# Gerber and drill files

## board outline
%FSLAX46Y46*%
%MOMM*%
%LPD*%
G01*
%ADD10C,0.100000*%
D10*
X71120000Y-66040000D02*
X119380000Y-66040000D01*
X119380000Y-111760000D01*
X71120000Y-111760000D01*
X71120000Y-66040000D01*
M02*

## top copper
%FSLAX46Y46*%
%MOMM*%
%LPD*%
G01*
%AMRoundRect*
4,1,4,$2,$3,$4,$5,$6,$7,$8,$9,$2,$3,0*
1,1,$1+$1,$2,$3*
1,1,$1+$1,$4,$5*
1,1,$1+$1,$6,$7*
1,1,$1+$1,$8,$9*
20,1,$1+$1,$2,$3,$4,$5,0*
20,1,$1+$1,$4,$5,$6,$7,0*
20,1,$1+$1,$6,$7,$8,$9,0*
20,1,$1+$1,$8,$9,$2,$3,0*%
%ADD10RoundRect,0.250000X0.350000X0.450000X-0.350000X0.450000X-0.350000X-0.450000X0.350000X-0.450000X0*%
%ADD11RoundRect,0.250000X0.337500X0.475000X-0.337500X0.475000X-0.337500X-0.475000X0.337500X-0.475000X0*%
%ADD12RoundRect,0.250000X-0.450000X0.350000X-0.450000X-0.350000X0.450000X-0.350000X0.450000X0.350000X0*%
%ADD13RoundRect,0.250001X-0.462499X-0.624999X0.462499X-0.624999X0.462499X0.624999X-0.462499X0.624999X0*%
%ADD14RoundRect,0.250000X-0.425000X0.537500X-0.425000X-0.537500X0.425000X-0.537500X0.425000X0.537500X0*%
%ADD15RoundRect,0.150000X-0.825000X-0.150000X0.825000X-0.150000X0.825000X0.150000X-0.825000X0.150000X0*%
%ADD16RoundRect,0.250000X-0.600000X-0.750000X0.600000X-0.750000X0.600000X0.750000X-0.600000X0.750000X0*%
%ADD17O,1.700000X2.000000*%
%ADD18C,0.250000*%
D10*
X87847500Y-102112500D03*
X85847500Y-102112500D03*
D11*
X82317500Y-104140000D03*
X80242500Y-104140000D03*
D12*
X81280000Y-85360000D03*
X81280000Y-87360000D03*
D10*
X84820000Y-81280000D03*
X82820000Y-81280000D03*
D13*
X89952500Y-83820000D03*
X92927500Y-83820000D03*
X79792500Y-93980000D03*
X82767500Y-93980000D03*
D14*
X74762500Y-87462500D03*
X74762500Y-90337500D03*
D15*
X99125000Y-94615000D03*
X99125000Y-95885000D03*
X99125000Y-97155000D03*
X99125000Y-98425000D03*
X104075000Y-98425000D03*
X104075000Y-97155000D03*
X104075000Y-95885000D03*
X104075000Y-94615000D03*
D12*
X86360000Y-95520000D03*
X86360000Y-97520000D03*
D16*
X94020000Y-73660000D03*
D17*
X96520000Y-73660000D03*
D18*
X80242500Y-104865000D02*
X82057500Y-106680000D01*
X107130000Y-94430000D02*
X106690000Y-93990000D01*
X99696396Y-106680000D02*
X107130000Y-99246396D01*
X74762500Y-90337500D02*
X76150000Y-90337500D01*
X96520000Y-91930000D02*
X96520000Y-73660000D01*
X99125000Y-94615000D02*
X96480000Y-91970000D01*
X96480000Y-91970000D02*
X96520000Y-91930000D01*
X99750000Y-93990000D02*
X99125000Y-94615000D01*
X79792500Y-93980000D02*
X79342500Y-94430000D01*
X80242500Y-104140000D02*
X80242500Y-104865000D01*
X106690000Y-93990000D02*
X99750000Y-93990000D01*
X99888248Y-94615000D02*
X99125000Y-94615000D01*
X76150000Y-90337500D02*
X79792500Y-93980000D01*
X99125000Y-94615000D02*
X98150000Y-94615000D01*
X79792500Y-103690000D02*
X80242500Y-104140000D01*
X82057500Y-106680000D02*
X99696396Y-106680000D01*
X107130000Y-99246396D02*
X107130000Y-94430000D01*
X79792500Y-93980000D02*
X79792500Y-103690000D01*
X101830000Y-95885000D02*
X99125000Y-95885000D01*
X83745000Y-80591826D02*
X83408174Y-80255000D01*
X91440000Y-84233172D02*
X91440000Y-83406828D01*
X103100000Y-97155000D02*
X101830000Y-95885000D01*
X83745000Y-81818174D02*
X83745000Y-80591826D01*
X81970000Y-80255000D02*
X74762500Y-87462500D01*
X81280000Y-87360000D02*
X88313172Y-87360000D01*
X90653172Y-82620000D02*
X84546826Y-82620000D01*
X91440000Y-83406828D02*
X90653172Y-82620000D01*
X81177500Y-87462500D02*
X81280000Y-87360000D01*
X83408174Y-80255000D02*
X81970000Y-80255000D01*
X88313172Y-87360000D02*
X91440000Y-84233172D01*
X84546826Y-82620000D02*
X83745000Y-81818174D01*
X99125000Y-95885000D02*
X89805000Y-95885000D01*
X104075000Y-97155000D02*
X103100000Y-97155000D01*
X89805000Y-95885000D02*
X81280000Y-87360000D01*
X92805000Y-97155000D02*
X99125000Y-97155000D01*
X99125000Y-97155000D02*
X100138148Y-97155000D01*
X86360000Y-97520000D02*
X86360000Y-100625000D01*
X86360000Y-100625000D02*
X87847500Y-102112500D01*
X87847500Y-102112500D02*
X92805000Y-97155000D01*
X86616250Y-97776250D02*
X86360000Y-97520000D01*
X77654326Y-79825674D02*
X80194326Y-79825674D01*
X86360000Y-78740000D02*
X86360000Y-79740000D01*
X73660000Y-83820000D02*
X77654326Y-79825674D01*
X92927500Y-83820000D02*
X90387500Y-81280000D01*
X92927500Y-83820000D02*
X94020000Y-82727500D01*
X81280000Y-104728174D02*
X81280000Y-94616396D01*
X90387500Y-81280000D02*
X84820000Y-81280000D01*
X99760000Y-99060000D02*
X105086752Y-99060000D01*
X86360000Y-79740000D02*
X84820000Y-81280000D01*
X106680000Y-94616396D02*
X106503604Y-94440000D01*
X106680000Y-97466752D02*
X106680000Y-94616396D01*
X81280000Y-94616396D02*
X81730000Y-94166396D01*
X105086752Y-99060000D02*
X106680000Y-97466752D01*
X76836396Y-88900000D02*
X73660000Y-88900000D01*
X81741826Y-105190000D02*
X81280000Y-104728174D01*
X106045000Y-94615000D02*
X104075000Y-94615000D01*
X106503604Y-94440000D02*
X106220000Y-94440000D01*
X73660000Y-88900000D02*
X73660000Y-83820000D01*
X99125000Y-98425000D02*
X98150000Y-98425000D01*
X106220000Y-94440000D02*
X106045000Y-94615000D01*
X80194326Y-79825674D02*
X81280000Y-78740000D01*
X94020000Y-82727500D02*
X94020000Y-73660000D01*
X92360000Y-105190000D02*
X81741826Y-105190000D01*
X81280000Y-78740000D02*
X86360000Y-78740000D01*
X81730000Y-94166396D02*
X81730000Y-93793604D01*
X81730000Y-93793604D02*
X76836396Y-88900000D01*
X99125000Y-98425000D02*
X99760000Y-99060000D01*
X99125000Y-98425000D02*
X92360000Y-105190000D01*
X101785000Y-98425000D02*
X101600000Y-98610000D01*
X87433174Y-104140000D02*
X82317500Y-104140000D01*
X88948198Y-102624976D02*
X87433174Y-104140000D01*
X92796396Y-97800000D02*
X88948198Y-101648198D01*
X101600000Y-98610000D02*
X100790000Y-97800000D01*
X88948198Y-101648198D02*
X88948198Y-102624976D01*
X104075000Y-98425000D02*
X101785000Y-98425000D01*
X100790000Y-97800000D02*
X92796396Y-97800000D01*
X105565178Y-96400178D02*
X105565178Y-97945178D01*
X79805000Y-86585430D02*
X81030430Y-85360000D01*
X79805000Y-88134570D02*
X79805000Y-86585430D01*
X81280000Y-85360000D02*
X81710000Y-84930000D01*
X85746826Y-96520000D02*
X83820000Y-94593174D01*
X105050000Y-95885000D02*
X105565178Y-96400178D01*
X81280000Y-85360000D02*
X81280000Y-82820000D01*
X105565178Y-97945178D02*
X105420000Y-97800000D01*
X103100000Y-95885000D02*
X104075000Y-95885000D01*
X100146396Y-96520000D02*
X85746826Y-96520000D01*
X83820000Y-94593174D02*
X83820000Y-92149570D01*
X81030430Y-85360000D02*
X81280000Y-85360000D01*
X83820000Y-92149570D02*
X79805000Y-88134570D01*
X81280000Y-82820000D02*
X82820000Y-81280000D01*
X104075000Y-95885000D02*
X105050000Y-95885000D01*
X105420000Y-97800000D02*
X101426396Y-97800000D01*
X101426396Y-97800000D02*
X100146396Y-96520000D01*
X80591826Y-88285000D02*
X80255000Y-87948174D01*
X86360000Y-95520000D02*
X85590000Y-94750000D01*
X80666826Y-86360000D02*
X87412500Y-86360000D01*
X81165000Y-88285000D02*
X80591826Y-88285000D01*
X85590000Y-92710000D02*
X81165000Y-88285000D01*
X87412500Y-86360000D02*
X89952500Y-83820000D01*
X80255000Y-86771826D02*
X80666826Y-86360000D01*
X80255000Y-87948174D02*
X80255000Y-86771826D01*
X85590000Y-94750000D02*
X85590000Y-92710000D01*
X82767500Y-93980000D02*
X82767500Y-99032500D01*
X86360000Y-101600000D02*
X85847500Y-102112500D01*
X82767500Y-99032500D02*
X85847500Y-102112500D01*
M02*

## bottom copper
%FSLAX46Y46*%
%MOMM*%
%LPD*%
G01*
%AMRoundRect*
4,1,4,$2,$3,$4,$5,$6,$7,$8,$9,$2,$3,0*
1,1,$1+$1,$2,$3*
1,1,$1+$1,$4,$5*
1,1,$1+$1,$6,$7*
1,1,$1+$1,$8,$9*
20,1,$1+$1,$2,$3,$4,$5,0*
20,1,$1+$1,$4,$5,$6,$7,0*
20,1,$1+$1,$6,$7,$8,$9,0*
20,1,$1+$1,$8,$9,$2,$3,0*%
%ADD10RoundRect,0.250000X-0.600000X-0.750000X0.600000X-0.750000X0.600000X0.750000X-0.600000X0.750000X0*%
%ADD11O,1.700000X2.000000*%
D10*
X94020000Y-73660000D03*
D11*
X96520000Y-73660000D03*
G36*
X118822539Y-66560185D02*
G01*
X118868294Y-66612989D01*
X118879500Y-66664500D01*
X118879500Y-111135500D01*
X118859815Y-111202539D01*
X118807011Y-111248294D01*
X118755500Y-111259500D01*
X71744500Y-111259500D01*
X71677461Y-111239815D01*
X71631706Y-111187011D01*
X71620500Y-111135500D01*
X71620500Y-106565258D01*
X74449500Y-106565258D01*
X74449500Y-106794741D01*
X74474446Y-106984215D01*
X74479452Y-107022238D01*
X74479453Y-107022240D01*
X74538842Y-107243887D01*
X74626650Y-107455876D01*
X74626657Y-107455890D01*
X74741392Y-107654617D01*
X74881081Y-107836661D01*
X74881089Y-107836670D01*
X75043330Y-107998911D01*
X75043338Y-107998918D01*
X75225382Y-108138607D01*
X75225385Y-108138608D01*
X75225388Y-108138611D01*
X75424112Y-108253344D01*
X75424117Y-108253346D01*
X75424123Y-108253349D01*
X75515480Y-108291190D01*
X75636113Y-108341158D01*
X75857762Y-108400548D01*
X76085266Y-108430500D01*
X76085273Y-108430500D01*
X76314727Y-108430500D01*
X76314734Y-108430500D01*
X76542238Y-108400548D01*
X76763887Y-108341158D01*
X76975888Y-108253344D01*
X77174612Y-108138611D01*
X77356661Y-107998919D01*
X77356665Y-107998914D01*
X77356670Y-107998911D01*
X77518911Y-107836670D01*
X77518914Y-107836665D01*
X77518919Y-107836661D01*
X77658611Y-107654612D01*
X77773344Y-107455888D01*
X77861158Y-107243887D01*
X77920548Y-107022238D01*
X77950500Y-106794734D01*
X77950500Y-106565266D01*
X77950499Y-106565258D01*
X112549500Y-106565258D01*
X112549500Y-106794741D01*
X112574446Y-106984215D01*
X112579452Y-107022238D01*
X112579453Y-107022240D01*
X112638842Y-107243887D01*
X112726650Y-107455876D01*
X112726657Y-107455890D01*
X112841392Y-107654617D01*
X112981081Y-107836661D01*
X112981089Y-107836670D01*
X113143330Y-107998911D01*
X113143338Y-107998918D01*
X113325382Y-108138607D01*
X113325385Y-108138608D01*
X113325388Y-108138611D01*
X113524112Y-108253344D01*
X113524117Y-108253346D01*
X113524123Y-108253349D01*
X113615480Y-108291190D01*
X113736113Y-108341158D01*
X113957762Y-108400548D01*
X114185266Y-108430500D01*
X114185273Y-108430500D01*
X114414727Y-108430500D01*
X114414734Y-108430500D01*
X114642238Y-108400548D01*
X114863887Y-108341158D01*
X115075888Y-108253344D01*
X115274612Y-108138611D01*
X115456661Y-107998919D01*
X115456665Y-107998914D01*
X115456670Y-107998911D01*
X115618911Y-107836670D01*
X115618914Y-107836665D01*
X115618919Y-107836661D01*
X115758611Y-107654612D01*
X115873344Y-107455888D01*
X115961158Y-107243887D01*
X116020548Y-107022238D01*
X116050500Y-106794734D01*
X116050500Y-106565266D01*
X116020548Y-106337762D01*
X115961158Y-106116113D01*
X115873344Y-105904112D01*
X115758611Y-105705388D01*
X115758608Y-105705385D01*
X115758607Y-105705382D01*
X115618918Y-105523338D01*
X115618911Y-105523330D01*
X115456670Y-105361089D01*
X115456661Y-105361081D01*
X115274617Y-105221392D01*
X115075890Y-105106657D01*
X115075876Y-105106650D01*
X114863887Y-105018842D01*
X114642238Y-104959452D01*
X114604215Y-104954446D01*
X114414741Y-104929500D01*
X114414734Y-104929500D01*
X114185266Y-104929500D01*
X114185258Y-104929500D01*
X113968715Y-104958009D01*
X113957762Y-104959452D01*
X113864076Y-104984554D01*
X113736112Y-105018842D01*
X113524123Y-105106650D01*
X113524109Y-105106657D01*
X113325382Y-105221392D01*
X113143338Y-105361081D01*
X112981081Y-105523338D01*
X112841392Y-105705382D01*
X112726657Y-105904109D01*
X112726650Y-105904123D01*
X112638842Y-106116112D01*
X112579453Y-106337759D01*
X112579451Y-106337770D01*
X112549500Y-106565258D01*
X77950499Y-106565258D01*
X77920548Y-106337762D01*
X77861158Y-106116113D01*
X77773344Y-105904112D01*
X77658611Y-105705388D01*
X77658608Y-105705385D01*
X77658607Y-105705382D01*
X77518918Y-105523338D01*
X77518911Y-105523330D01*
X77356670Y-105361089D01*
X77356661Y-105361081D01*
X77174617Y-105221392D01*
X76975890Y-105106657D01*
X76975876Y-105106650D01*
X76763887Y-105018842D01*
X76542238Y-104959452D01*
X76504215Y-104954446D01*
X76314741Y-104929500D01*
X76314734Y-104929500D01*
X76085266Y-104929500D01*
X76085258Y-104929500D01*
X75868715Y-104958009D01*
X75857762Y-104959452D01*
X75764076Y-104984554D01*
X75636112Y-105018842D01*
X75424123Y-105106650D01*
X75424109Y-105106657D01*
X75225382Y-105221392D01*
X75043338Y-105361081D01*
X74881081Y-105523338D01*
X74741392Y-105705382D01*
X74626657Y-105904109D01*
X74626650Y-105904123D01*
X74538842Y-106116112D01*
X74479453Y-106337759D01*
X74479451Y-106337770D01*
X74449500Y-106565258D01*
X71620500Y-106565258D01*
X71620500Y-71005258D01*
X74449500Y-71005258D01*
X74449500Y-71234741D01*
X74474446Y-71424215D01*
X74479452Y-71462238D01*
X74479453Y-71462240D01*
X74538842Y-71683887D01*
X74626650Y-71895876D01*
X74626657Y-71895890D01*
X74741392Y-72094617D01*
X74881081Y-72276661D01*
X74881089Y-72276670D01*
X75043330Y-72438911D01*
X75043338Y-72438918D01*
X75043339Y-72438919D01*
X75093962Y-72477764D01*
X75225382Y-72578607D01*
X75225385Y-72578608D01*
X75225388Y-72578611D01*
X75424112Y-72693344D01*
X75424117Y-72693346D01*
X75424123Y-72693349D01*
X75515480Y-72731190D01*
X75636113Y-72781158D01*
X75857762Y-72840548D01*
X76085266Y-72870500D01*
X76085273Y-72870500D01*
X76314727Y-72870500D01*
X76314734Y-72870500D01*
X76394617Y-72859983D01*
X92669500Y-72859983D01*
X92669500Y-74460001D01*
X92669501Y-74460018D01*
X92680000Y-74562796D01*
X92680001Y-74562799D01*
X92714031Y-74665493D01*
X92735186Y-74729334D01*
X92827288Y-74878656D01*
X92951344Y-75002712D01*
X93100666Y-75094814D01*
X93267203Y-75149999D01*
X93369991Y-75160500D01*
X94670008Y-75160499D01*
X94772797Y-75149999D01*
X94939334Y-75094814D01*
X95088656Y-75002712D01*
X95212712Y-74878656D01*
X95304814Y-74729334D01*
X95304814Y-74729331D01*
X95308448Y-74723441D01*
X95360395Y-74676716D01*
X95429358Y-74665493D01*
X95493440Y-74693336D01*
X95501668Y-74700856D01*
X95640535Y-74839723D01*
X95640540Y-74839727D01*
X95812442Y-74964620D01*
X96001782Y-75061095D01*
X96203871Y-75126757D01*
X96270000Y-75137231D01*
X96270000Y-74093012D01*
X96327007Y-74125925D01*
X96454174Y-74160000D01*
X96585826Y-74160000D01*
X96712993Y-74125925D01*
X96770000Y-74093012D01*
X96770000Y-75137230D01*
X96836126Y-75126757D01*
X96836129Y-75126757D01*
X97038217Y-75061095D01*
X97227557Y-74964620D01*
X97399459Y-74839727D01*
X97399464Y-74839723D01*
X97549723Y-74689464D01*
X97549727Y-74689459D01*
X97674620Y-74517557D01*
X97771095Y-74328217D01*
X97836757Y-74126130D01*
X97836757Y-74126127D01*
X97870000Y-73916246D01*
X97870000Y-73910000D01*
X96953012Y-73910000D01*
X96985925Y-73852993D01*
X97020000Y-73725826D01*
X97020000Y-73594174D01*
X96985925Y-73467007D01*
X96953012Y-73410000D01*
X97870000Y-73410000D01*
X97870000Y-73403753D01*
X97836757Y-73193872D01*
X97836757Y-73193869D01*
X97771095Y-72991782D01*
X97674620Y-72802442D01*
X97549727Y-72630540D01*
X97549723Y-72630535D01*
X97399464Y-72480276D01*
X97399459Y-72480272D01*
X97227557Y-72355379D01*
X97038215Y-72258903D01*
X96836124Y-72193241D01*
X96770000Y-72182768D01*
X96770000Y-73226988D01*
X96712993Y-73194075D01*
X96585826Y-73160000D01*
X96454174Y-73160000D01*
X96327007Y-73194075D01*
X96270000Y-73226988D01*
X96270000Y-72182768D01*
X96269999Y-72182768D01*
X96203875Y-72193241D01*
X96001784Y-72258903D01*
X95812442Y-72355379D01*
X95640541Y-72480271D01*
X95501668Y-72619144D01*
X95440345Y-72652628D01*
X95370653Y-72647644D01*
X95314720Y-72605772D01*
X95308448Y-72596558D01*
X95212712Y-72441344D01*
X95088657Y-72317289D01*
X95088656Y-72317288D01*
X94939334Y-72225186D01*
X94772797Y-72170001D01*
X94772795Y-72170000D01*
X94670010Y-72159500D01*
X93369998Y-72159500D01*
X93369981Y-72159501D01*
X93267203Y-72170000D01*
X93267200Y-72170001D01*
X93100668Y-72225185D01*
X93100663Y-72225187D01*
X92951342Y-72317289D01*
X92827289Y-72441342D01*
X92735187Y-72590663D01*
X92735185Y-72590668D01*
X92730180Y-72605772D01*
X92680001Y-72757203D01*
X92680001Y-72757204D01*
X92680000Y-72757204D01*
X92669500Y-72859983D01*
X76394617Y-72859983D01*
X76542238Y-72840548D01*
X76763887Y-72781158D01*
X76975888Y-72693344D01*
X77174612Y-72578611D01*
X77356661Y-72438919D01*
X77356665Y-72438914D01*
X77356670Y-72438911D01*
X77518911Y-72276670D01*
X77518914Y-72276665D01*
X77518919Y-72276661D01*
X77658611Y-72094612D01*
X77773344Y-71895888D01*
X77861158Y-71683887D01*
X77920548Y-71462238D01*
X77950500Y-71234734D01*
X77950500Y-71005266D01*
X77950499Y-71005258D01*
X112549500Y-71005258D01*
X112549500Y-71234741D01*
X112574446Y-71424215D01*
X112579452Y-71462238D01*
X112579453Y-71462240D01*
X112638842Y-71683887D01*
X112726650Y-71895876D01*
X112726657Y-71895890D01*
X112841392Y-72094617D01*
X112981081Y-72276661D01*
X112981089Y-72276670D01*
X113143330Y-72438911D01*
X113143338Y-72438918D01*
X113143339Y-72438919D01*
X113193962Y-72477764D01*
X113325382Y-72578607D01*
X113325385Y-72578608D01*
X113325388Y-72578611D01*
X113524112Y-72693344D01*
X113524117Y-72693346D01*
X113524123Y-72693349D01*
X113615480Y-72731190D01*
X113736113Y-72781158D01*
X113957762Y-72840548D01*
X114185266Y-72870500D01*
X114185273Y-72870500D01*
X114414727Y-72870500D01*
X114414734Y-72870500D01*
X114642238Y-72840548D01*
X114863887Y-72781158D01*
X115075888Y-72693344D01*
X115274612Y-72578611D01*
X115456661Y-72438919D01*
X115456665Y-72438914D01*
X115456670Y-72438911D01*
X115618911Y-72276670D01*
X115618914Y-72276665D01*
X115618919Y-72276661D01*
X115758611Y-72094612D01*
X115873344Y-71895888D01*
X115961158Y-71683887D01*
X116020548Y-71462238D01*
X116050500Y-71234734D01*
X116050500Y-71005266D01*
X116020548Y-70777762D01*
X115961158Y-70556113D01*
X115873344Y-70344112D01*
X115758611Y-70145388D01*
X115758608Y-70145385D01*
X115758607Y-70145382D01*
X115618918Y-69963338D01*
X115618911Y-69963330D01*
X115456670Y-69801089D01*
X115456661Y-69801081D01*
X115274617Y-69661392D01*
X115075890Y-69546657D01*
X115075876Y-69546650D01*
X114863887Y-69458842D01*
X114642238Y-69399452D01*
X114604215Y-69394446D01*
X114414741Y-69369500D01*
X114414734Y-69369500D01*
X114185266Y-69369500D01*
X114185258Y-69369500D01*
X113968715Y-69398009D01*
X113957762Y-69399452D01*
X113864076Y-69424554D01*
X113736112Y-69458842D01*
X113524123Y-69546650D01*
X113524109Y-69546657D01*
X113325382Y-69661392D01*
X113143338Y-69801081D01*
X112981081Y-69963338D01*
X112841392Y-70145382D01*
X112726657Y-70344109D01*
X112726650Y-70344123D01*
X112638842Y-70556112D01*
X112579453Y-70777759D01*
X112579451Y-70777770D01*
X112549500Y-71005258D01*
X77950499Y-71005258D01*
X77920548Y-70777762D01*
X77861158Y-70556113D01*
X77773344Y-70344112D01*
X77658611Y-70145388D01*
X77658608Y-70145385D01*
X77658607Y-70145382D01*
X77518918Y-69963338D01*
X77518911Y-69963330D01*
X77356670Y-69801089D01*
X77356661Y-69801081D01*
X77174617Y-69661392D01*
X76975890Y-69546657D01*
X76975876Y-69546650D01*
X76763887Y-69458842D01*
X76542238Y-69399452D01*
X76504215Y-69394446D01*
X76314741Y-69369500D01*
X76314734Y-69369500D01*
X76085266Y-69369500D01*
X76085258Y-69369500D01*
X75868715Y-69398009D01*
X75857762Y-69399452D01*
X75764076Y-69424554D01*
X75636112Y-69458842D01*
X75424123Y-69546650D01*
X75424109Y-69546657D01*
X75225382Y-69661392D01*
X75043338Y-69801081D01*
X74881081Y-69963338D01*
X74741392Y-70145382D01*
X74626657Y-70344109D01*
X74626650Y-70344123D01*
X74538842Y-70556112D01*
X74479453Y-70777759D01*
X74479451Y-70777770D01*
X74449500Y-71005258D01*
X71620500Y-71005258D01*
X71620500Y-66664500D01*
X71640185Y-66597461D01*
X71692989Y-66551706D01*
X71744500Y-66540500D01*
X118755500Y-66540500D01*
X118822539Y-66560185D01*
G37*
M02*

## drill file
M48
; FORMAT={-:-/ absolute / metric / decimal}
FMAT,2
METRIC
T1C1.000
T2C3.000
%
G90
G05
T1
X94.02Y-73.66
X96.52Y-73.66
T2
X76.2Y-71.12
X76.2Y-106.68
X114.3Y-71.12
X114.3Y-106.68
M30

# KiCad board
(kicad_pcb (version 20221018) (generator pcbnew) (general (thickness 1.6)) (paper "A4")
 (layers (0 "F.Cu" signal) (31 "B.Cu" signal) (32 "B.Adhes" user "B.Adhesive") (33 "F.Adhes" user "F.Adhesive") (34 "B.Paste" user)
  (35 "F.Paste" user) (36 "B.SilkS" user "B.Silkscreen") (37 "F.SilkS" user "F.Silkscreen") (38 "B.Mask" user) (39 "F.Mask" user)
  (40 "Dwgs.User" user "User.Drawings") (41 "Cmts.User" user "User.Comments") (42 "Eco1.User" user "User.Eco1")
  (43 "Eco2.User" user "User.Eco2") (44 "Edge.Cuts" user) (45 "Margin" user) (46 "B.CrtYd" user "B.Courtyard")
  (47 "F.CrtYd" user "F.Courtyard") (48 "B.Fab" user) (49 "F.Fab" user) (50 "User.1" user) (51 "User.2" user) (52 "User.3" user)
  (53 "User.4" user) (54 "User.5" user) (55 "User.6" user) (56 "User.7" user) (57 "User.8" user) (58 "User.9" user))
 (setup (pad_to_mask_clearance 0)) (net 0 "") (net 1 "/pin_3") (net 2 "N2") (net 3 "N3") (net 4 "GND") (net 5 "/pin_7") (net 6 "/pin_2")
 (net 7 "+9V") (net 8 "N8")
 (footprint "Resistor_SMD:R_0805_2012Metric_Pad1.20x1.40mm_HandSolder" (layer "F.Cu") (at 86.8475 102.1125 180)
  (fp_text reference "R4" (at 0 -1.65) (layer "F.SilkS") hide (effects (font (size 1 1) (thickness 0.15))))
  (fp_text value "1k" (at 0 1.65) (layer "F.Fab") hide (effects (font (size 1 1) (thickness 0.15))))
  (pad "1" smd roundrect (at -1 0 180) (size 1.2 1.4) (layers "F.Cu" "F.Paste" "F.Mask") (roundrect_rratio 0.208333) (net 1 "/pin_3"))
  (pad "2" smd roundrect (at 1 0 180) (size 1.2 1.4) (layers "F.Cu" "F.Paste" "F.Mask") (roundrect_rratio 0.208333) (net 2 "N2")))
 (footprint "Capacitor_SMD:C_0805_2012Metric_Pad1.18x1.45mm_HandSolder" (layer "F.Cu") (at 81.28 104.14 180)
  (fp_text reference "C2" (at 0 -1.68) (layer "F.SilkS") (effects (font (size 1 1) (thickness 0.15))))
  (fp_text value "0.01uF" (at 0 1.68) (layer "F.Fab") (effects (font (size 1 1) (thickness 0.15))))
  (pad "1" smd roundrect (at -1.0375 0 180) (size 1.175 1.45) (layers "F.Cu" "F.Paste" "F.Mask") (roundrect_rratio 0.212766) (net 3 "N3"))
  (pad "2" smd roundrect (at 1.0375 0 180) (size 1.175 1.45) (layers "F.Cu" "F.Paste" "F.Mask") (roundrect_rratio 0.212766) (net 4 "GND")))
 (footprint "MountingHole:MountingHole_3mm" (layer "F.Cu") (at 76.2 106.68)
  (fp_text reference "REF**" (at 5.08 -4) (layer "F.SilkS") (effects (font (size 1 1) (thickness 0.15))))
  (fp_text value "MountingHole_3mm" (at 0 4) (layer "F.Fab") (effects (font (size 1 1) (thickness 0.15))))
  (pad "" np_thru_hole circle (at 0 0) (size 3 3) (drill 3) (layers "F&B.Cu" "*.Mask")))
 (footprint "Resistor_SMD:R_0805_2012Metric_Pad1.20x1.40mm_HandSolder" (layer "F.Cu") (at 81.28 86.36 -90)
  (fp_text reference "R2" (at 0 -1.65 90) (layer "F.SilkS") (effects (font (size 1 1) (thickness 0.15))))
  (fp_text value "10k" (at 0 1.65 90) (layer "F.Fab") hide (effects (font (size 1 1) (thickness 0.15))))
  (pad "1" smd roundrect (at -1 0 270) (size 1.2 1.4) (layers "F.Cu" "F.Paste" "F.Mask") (roundrect_rratio 0.208333) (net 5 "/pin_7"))
  (pad "2" smd roundrect (at 1 0 270) (size 1.2 1.4) (layers "F.Cu" "F.Paste" "F.Mask") (roundrect_rratio 0.208333) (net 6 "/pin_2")))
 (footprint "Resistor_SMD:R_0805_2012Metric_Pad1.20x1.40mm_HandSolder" (layer "F.Cu") (at 83.82 81.28 180)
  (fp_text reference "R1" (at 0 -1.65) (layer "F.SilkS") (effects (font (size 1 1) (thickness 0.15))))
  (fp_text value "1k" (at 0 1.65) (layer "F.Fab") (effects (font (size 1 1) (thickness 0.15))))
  (pad "1" smd roundrect (at -1 0 180) (size 1.2 1.4) (layers "F.Cu" "F.Paste" "F.Mask") (roundrect_rratio 0.208333) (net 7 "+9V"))
  (pad "2" smd roundrect (at 1 0 180) (size 1.2 1.4) (layers "F.Cu" "F.Paste" "F.Mask") (roundrect_rratio 0.208333) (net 5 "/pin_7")))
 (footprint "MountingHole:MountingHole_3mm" (layer "F.Cu") (at 114.3 106.68)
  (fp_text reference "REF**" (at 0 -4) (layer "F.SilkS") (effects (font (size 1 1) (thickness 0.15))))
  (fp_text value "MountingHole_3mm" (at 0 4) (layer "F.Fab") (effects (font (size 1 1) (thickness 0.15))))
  (pad "" np_thru_hole circle (at 0 0) (size 3 3) (drill 3) (layers "F&B.Cu" "*.Mask")))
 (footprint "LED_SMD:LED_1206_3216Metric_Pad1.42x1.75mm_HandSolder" (layer "F.Cu") (at 91.44 83.82)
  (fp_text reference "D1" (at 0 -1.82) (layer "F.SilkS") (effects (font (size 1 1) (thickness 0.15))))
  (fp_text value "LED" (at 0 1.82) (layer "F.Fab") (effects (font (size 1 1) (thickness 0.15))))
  (pad "1" smd roundrect (at -1.4875 0) (size 1.425 1.75) (layers "F.Cu" "F.Paste" "F.Mask") (roundrect_rratio 0.175439) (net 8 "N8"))
  (pad "2" smd roundrect (at 1.4875 0) (size 1.425 1.75) (layers "F.Cu" "F.Paste" "F.Mask") (roundrect_rratio 0.175439) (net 7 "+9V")))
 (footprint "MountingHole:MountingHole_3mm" (layer "F.Cu") (at 76.2 71.12)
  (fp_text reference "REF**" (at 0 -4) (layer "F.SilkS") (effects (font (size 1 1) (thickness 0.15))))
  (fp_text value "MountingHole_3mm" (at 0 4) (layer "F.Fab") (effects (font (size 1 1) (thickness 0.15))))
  (pad "" np_thru_hole circle (at 0 0) (size 3 3) (drill 3) (layers "*.Cu" "*.Mask")))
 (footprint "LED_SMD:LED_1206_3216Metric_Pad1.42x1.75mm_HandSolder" (layer "F.Cu") (at 81.28 93.98)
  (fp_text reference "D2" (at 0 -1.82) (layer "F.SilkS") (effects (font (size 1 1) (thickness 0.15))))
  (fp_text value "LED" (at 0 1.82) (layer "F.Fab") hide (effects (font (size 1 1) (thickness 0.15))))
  (pad "1" smd roundrect (at -1.4875 0) (size 1.425 1.75) (layers "F.Cu" "F.Paste" "F.Mask") (roundrect_rratio 0.175439) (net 4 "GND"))
  (pad "2" smd roundrect (at 1.4875 0) (size 1.425 1.75) (layers "F.Cu" "F.Paste" "F.Mask") (roundrect_rratio 0.175439) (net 2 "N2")))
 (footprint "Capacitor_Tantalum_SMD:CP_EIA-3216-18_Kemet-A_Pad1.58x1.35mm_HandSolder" (layer "F.Cu") (at 74.7625 88.9 -90)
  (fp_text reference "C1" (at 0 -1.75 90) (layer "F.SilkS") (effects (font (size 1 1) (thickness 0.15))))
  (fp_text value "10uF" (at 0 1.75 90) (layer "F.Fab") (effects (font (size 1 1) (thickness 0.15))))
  (pad "1" smd roundrect (at -1.4375 0 270) (size 1.575 1.35) (layers "F.Cu" "F.Paste" "F.Mask") (roundrect_rratio 0.185185)
   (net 6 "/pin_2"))
  (pad "2" smd roundrect (at 1.4375 0 270) (size 1.575 1.35) (layers "F.Cu" "F.Paste" "F.Mask") (roundrect_rratio 0.185185) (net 4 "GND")))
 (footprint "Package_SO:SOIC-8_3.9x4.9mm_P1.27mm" (layer "F.Cu") (at 101.6 96.52)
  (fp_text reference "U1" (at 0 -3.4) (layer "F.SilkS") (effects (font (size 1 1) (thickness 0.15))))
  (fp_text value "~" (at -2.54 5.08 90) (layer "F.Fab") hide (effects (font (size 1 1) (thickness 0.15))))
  (pad "1" smd roundrect (at -2.475 -1.905) (size 1.95 0.6) (layers "F.Cu" "F.Paste" "F.Mask") (roundrect_rratio 0.25) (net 4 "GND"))
  (pad "2" smd roundrect (at -2.475 -0.635) (size 1.95 0.6) (layers "F.Cu" "F.Paste" "F.Mask") (roundrect_rratio 0.25) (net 6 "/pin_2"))
  (pad "3" smd roundrect (at -2.475 0.635) (size 1.95 0.6) (layers "F.Cu" "F.Paste" "F.Mask") (roundrect_rratio 0.25) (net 1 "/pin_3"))
  (pad "4" smd roundrect (at -2.475 1.905) (size 1.95 0.6) (layers "F.Cu" "F.Paste" "F.Mask") (roundrect_rratio 0.25) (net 7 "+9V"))
  (pad "5" smd roundrect (at 2.475 1.905) (size 1.95 0.6) (layers "F.Cu" "F.Paste" "F.Mask") (roundrect_rratio 0.25) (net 3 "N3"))
  (pad "6" smd roundrect (at 2.475 0.635) (size 1.95 0.6) (layers "F.Cu" "F.Paste" "F.Mask") (roundrect_rratio 0.25) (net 6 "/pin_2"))
  (pad "7" smd roundrect (at 2.475 -0.635) (size 1.95 0.6) (layers "F.Cu" "F.Paste" "F.Mask") (roundrect_rratio 0.25) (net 5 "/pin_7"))
  (pad "8" smd roundrect (at 2.475 -1.905) (size 1.95 0.6) (layers "F.Cu" "F.Paste" "F.Mask") (roundrect_rratio 0.25) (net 7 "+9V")))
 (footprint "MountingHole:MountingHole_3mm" (layer "F.Cu") (at 114.3 71.12)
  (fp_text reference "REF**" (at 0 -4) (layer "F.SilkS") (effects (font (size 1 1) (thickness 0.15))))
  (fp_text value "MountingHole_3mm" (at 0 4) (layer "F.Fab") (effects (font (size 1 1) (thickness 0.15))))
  (pad "" np_thru_hole circle (at 0 0) (size 3 3) (drill 3) (layers "F&B.Cu" "*.Mask")))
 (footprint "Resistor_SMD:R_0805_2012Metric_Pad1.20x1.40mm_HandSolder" (layer "F.Cu") (at 86.36 96.52 -90)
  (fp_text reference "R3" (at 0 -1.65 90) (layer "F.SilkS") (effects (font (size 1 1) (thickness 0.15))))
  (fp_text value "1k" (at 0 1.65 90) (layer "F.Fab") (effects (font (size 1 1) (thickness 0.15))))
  (pad "1" smd roundrect (at -1 0 270) (size 1.2 1.4) (layers "F.Cu" "F.Paste" "F.Mask") (roundrect_rratio 0.208333) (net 8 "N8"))
  (pad "2" smd roundrect (at 1 0 270) (size 1.2 1.4) (layers "F.Cu" "F.Paste" "F.Mask") (roundrect_rratio 0.208333) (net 1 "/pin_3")))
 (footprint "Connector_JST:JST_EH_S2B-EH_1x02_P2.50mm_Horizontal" (layer "F.Cu") (at 94.02 73.66)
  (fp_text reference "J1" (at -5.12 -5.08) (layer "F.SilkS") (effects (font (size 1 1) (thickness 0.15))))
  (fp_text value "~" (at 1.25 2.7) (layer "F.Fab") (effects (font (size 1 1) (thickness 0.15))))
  (pad "1" thru_hole roundrect (at 0 0) (size 1.7 2) (drill 1) (layers "*.Cu" "*.Mask") (roundrect_rratio 0.147059) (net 7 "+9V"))
  (pad "2" thru_hole oval (at 2.5 0) (size 1.7 2) (drill 1) (layers "*.Cu" "*.Mask") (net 4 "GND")))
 (gr_rect (start 71.12 66.04) (end 119.38 111.76) (stroke (width 0.1) (type default)) (fill none) (layer "Edge.Cuts"))
 (segment (start 80.2425 104.865) (end 82.0575 106.68) (width 0.25) (layer "F.Cu") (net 4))
 (segment (start 107.13 94.43) (end 106.69 93.99) (width 0.25) (layer "F.Cu") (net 4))
 (segment (start 99.696396 106.68) (end 107.13 99.246396) (width 0.25) (layer "F.Cu") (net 4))
 (segment (start 74.7625 90.3375) (end 76.15 90.3375) (width 0.25) (layer "F.Cu") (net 4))
 (segment (start 96.52 91.93) (end 96.52 73.66) (width 0.25) (layer "F.Cu") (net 4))
 (segment (start 99.125 94.615) (end 96.48 91.97) (width 0.25) (layer "F.Cu") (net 4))
 (segment (start 96.48 91.97) (end 96.52 91.93) (width 0.25) (layer "F.Cu") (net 4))
 (segment (start 99.75 93.99) (end 99.125 94.615) (width 0.25) (layer "F.Cu") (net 4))
 (segment (start 79.7925 93.98) (end 79.3425 94.43) (width 0.25) (layer "F.Cu") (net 4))
 (segment (start 80.2425 104.14) (end 80.2425 104.865) (width 0.25) (layer "F.Cu") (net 4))
 (segment (start 106.69 93.99) (end 99.75 93.99) (width 0.25) (layer "F.Cu") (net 4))
 (segment (start 99.888248 94.615) (end 99.125 94.615) (width 0.25) (layer "F.Cu") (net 4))
 (segment (start 76.15 90.3375) (end 79.7925 93.98) (width 0.25) (layer "F.Cu") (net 4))
 (segment (start 99.125 94.615) (end 98.15 94.615) (width 0.25) (layer "F.Cu") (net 4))
 (segment (start 79.7925 103.69) (end 80.2425 104.14) (width 0.25) (layer "F.Cu") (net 4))
 (segment (start 82.0575 106.68) (end 99.696396 106.68) (width 0.25) (layer "F.Cu") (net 4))
 (segment (start 107.13 99.246396) (end 107.13 94.43) (width 0.25) (layer "F.Cu") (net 4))
 (segment (start 79.7925 93.98) (end 79.7925 103.69) (width 0.25) (layer "F.Cu") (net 4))
 (segment (start 101.83 95.885) (end 99.125 95.885) (width 0.25) (layer "F.Cu") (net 6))
 (segment (start 83.745 80.591826) (end 83.408174 80.255) (width 0.25) (layer "F.Cu") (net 6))
 (segment (start 91.44 84.233172) (end 91.44 83.406828) (width 0.25) (layer "F.Cu") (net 6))
 (segment (start 103.1 97.155) (end 101.83 95.885) (width 0.25) (layer "F.Cu") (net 6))
 (segment (start 83.745 81.818174) (end 83.745 80.591826) (width 0.25) (layer "F.Cu") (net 6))
 (segment (start 81.97 80.255) (end 74.7625 87.4625) (width 0.25) (layer "F.Cu") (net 6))
 (segment (start 81.28 87.36) (end 88.313172 87.36) (width 0.25) (layer "F.Cu") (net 6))
 (segment (start 90.653172 82.62) (end 84.546826 82.62) (width 0.25) (layer "F.Cu") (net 6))
 (segment (start 91.44 83.406828) (end 90.653172 82.62) (width 0.25) (layer "F.Cu") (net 6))
 (segment (start 81.1775 87.4625) (end 81.28 87.36) (width 0.25) (layer "F.Cu") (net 6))
 (segment (start 83.408174 80.255) (end 81.97 80.255) (width 0.25) (layer "F.Cu") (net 6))
 (segment (start 88.313172 87.36) (end 91.44 84.233172) (width 0.25) (layer "F.Cu") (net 6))
 (segment (start 84.546826 82.62) (end 83.745 81.818174) (width 0.25) (layer "F.Cu") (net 6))
 (segment (start 99.125 95.885) (end 89.805 95.885) (width 0.25) (layer "F.Cu") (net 6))
 (segment (start 104.075 97.155) (end 103.1 97.155) (width 0.25) (layer "F.Cu") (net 6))
 (segment (start 89.805 95.885) (end 81.28 87.36) (width 0.25) (layer "F.Cu") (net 6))
 (segment (start 92.805 97.155) (end 99.125 97.155) (width 0.25) (layer "F.Cu") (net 1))
 (segment (start 99.125 97.155) (end 100.138148 97.155) (width 0.25) (layer "F.Cu") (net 1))
 (segment (start 86.36 97.52) (end 86.36 100.625) (width 0.25) (layer "F.Cu") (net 1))
 (segment (start 86.36 100.625) (end 87.8475 102.1125) (width 0.25) (layer "F.Cu") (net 1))
 (segment (start 87.8475 102.1125) (end 92.805 97.155) (width 0.25) (layer "F.Cu") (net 1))
 (segment (start 86.61625 97.77625) (end 86.36 97.52) (width 0.25) (layer "F.Cu") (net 1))
 (segment (start 77.654326 79.825674) (end 80.194326 79.825674) (width 0.25) (layer "F.Cu") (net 7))
 (segment (start 86.36 78.74) (end 86.36 79.74) (width 0.25) (layer "F.Cu") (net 7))
 (segment (start 73.66 83.82) (end 77.654326 79.825674) (width 0.25) (layer "F.Cu") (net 7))
 (segment (start 92.9275 83.82) (end 90.3875 81.28) (width 0.25) (layer "F.Cu") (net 7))
 (segment (start 92.9275 83.82) (end 94.02 82.7275) (width 0.25) (layer "F.Cu") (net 7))
 (segment (start 81.28 104.728174) (end 81.28 94.616396) (width 0.25) (layer "F.Cu") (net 7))
 (segment (start 90.3875 81.28) (end 84.82 81.28) (width 0.25) (layer "F.Cu") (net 7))
 (segment (start 99.76 99.06) (end 105.086752 99.06) (width 0.25) (layer "F.Cu") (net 7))
 (segment (start 86.36 79.74) (end 84.82 81.28) (width 0.25) (layer "F.Cu") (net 7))
 (segment (start 106.68 94.616396) (end 106.503604 94.44) (width 0.25) (layer "F.Cu") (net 7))
 (segment (start 106.68 97.466752) (end 106.68 94.616396) (width 0.25) (layer "F.Cu") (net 7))
 (segment (start 81.28 94.616396) (end 81.73 94.166396) (width 0.25) (layer "F.Cu") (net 7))
 (segment (start 105.086752 99.06) (end 106.68 97.466752) (width 0.25) (layer "F.Cu") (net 7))
 (segment (start 76.836396 88.9) (end 73.66 88.9) (width 0.25) (layer "F.Cu") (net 7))
 (segment (start 81.741826 105.19) (end 81.28 104.728174) (width 0.25) (layer "F.Cu") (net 7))
 (segment (start 106.045 94.615) (end 104.075 94.615) (width 0.25) (layer "F.Cu") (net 7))
 (segment (start 106.503604 94.44) (end 106.22 94.44) (width 0.25) (layer "F.Cu") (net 7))
 (segment (start 73.66 88.9) (end 73.66 83.82) (width 0.25) (layer "F.Cu") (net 7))
 (segment (start 99.125 98.425) (end 98.15 98.425) (width 0.25) (layer "F.Cu") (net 7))
 (segment (start 106.22 94.44) (end 106.045 94.615) (width 0.25) (layer "F.Cu") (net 7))
 (segment (start 80.194326 79.825674) (end 81.28 78.74) (width 0.25) (layer "F.Cu") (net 7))
 (segment (start 94.02 82.7275) (end 94.02 73.66) (width 0.25) (layer "F.Cu") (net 7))
 (segment (start 92.36 105.19) (end 81.741826 105.19) (width 0.25) (layer "F.Cu") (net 7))
 (segment (start 81.28 78.74) (end 86.36 78.74) (width 0.25) (layer "F.Cu") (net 7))
 (segment (start 81.73 94.166396) (end 81.73 93.793604) (width 0.25) (layer "F.Cu") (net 7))
 (segment (start 81.73 93.793604) (end 76.836396 88.9) (width 0.25) (layer "F.Cu") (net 7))
 (segment (start 99.125 98.425) (end 99.76 99.06) (width 0.25) (layer "F.Cu") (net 7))
 (segment (start 99.125 98.425) (end 92.36 105.19) (width 0.25) (layer "F.Cu") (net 7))
 (segment (start 101.785 98.425) (end 101.6 98.61) (width 0.25) (layer "F.Cu") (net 3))
 (segment (start 87.433174 104.14) (end 82.3175 104.14) (width 0.25) (layer "F.Cu") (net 3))
 (segment (start 88.948198 102.624976) (end 87.433174 104.14) (width 0.25) (layer "F.Cu") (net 3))
 (segment (start 92.796396 97.8) (end 88.948198 101.648198) (width 0.25) (layer "F.Cu") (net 3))
 (segment (start 101.6 98.61) (end 100.79 97.8) (width 0.25) (layer "F.Cu") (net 3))
 (segment (start 88.948198 101.648198) (end 88.948198 102.624976) (width 0.25) (layer "F.Cu") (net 3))
 (segment (start 104.075 98.425) (end 101.785 98.425) (width 0.25) (layer "F.Cu") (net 3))
 (segment (start 100.79 97.8) (end 92.796396 97.8) (width 0.25) (layer "F.Cu") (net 3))
 (segment (start 105.565178 96.400178) (end 105.565178 97.945178) (width 0.25) (layer "F.Cu") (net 5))
 (segment (start 79.805 86.58543) (end 81.03043 85.36) (width 0.25) (layer "F.Cu") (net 5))
 (segment (start 79.805 88.13457) (end 79.805 86.58543) (width 0.25) (layer "F.Cu") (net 5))
 (segment (start 81.28 85.36) (end 81.71 84.93) (width 0.25) (layer "F.Cu") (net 5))
 (segment (start 85.746826 96.52) (end 83.82 94.593174) (width 0.25) (layer "F.Cu") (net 5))
 (segment (start 105.05 95.885) (end 105.565178 96.400178) (width 0.25) (layer "F.Cu") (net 5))
 (segment (start 81.28 85.36) (end 81.28 82.82) (width 0.25) (layer "F.Cu") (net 5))
 (segment (start 105.565178 97.945178) (end 105.42 97.8) (width 0.25) (layer "F.Cu") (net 5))
 (segment (start 103.1 95.885) (end 104.075 95.885) (width 0.25) (layer "F.Cu") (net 5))
 (segment (start 100.146396 96.52) (end 85.746826 96.52) (width 0.25) (layer "F.Cu") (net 5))
 (segment (start 83.82 94.593174) (end 83.82 92.14957) (width 0.25) (layer "F.Cu") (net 5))
 (segment (start 81.03043 85.36) (end 81.28 85.36) (width 0.25) (layer "F.Cu") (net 5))
 (segment (start 83.82 92.14957) (end 79.805 88.13457) (width 0.25) (layer "F.Cu") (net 5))
 (segment (start 81.28 82.82) (end 82.82 81.28) (width 0.25) (layer "F.Cu") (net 5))
 (segment (start 104.075 95.885) (end 105.05 95.885) (width 0.25) (layer "F.Cu") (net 5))
 (segment (start 105.42 97.8) (end 101.426396 97.8) (width 0.25) (layer "F.Cu") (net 5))
 (segment (start 101.426396 97.8) (end 100.146396 96.52) (width 0.25) (layer "F.Cu") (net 5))
 (segment (start 80.591826 88.285) (end 80.255 87.948174) (width 0.25) (layer "F.Cu") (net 8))
 (segment (start 86.36 95.52) (end 85.59 94.75) (width 0.25) (layer "F.Cu") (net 8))
 (segment (start 80.666826 86.36) (end 87.4125 86.36) (width 0.25) (layer "F.Cu") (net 8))
 (segment (start 81.165 88.285) (end 80.591826 88.285) (width 0.25) (layer "F.Cu") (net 8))
 (segment (start 85.59 92.71) (end 81.165 88.285) (width 0.25) (layer "F.Cu") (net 8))
 (segment (start 87.4125 86.36) (end 89.9525 83.82) (width 0.25) (layer "F.Cu") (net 8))
 (segment (start 80.255 86.771826) (end 80.666826 86.36) (width 0.25) (layer "F.Cu") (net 8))
 (segment (start 80.255 87.948174) (end 80.255 86.771826) (width 0.25) (layer "F.Cu") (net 8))
 (segment (start 85.59 94.75) (end 85.59 92.71) (width 0.25) (layer "F.Cu") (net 8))
 (segment (start 82.7675 93.98) (end 82.7675 99.0325) (width 0.25) (layer "F.Cu") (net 2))
 (segment (start 86.36 101.6) (end 85.8475 102.1125) (width 0.25) (layer "F.Cu") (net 2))
 (segment (start 82.7675 99.0325) (end 85.8475 102.1125) (width 0.25) (layer "F.Cu") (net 2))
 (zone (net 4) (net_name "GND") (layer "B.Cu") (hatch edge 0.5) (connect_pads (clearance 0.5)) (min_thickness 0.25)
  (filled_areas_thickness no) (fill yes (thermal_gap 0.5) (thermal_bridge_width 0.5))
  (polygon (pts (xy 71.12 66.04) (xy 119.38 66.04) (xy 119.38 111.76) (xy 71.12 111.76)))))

